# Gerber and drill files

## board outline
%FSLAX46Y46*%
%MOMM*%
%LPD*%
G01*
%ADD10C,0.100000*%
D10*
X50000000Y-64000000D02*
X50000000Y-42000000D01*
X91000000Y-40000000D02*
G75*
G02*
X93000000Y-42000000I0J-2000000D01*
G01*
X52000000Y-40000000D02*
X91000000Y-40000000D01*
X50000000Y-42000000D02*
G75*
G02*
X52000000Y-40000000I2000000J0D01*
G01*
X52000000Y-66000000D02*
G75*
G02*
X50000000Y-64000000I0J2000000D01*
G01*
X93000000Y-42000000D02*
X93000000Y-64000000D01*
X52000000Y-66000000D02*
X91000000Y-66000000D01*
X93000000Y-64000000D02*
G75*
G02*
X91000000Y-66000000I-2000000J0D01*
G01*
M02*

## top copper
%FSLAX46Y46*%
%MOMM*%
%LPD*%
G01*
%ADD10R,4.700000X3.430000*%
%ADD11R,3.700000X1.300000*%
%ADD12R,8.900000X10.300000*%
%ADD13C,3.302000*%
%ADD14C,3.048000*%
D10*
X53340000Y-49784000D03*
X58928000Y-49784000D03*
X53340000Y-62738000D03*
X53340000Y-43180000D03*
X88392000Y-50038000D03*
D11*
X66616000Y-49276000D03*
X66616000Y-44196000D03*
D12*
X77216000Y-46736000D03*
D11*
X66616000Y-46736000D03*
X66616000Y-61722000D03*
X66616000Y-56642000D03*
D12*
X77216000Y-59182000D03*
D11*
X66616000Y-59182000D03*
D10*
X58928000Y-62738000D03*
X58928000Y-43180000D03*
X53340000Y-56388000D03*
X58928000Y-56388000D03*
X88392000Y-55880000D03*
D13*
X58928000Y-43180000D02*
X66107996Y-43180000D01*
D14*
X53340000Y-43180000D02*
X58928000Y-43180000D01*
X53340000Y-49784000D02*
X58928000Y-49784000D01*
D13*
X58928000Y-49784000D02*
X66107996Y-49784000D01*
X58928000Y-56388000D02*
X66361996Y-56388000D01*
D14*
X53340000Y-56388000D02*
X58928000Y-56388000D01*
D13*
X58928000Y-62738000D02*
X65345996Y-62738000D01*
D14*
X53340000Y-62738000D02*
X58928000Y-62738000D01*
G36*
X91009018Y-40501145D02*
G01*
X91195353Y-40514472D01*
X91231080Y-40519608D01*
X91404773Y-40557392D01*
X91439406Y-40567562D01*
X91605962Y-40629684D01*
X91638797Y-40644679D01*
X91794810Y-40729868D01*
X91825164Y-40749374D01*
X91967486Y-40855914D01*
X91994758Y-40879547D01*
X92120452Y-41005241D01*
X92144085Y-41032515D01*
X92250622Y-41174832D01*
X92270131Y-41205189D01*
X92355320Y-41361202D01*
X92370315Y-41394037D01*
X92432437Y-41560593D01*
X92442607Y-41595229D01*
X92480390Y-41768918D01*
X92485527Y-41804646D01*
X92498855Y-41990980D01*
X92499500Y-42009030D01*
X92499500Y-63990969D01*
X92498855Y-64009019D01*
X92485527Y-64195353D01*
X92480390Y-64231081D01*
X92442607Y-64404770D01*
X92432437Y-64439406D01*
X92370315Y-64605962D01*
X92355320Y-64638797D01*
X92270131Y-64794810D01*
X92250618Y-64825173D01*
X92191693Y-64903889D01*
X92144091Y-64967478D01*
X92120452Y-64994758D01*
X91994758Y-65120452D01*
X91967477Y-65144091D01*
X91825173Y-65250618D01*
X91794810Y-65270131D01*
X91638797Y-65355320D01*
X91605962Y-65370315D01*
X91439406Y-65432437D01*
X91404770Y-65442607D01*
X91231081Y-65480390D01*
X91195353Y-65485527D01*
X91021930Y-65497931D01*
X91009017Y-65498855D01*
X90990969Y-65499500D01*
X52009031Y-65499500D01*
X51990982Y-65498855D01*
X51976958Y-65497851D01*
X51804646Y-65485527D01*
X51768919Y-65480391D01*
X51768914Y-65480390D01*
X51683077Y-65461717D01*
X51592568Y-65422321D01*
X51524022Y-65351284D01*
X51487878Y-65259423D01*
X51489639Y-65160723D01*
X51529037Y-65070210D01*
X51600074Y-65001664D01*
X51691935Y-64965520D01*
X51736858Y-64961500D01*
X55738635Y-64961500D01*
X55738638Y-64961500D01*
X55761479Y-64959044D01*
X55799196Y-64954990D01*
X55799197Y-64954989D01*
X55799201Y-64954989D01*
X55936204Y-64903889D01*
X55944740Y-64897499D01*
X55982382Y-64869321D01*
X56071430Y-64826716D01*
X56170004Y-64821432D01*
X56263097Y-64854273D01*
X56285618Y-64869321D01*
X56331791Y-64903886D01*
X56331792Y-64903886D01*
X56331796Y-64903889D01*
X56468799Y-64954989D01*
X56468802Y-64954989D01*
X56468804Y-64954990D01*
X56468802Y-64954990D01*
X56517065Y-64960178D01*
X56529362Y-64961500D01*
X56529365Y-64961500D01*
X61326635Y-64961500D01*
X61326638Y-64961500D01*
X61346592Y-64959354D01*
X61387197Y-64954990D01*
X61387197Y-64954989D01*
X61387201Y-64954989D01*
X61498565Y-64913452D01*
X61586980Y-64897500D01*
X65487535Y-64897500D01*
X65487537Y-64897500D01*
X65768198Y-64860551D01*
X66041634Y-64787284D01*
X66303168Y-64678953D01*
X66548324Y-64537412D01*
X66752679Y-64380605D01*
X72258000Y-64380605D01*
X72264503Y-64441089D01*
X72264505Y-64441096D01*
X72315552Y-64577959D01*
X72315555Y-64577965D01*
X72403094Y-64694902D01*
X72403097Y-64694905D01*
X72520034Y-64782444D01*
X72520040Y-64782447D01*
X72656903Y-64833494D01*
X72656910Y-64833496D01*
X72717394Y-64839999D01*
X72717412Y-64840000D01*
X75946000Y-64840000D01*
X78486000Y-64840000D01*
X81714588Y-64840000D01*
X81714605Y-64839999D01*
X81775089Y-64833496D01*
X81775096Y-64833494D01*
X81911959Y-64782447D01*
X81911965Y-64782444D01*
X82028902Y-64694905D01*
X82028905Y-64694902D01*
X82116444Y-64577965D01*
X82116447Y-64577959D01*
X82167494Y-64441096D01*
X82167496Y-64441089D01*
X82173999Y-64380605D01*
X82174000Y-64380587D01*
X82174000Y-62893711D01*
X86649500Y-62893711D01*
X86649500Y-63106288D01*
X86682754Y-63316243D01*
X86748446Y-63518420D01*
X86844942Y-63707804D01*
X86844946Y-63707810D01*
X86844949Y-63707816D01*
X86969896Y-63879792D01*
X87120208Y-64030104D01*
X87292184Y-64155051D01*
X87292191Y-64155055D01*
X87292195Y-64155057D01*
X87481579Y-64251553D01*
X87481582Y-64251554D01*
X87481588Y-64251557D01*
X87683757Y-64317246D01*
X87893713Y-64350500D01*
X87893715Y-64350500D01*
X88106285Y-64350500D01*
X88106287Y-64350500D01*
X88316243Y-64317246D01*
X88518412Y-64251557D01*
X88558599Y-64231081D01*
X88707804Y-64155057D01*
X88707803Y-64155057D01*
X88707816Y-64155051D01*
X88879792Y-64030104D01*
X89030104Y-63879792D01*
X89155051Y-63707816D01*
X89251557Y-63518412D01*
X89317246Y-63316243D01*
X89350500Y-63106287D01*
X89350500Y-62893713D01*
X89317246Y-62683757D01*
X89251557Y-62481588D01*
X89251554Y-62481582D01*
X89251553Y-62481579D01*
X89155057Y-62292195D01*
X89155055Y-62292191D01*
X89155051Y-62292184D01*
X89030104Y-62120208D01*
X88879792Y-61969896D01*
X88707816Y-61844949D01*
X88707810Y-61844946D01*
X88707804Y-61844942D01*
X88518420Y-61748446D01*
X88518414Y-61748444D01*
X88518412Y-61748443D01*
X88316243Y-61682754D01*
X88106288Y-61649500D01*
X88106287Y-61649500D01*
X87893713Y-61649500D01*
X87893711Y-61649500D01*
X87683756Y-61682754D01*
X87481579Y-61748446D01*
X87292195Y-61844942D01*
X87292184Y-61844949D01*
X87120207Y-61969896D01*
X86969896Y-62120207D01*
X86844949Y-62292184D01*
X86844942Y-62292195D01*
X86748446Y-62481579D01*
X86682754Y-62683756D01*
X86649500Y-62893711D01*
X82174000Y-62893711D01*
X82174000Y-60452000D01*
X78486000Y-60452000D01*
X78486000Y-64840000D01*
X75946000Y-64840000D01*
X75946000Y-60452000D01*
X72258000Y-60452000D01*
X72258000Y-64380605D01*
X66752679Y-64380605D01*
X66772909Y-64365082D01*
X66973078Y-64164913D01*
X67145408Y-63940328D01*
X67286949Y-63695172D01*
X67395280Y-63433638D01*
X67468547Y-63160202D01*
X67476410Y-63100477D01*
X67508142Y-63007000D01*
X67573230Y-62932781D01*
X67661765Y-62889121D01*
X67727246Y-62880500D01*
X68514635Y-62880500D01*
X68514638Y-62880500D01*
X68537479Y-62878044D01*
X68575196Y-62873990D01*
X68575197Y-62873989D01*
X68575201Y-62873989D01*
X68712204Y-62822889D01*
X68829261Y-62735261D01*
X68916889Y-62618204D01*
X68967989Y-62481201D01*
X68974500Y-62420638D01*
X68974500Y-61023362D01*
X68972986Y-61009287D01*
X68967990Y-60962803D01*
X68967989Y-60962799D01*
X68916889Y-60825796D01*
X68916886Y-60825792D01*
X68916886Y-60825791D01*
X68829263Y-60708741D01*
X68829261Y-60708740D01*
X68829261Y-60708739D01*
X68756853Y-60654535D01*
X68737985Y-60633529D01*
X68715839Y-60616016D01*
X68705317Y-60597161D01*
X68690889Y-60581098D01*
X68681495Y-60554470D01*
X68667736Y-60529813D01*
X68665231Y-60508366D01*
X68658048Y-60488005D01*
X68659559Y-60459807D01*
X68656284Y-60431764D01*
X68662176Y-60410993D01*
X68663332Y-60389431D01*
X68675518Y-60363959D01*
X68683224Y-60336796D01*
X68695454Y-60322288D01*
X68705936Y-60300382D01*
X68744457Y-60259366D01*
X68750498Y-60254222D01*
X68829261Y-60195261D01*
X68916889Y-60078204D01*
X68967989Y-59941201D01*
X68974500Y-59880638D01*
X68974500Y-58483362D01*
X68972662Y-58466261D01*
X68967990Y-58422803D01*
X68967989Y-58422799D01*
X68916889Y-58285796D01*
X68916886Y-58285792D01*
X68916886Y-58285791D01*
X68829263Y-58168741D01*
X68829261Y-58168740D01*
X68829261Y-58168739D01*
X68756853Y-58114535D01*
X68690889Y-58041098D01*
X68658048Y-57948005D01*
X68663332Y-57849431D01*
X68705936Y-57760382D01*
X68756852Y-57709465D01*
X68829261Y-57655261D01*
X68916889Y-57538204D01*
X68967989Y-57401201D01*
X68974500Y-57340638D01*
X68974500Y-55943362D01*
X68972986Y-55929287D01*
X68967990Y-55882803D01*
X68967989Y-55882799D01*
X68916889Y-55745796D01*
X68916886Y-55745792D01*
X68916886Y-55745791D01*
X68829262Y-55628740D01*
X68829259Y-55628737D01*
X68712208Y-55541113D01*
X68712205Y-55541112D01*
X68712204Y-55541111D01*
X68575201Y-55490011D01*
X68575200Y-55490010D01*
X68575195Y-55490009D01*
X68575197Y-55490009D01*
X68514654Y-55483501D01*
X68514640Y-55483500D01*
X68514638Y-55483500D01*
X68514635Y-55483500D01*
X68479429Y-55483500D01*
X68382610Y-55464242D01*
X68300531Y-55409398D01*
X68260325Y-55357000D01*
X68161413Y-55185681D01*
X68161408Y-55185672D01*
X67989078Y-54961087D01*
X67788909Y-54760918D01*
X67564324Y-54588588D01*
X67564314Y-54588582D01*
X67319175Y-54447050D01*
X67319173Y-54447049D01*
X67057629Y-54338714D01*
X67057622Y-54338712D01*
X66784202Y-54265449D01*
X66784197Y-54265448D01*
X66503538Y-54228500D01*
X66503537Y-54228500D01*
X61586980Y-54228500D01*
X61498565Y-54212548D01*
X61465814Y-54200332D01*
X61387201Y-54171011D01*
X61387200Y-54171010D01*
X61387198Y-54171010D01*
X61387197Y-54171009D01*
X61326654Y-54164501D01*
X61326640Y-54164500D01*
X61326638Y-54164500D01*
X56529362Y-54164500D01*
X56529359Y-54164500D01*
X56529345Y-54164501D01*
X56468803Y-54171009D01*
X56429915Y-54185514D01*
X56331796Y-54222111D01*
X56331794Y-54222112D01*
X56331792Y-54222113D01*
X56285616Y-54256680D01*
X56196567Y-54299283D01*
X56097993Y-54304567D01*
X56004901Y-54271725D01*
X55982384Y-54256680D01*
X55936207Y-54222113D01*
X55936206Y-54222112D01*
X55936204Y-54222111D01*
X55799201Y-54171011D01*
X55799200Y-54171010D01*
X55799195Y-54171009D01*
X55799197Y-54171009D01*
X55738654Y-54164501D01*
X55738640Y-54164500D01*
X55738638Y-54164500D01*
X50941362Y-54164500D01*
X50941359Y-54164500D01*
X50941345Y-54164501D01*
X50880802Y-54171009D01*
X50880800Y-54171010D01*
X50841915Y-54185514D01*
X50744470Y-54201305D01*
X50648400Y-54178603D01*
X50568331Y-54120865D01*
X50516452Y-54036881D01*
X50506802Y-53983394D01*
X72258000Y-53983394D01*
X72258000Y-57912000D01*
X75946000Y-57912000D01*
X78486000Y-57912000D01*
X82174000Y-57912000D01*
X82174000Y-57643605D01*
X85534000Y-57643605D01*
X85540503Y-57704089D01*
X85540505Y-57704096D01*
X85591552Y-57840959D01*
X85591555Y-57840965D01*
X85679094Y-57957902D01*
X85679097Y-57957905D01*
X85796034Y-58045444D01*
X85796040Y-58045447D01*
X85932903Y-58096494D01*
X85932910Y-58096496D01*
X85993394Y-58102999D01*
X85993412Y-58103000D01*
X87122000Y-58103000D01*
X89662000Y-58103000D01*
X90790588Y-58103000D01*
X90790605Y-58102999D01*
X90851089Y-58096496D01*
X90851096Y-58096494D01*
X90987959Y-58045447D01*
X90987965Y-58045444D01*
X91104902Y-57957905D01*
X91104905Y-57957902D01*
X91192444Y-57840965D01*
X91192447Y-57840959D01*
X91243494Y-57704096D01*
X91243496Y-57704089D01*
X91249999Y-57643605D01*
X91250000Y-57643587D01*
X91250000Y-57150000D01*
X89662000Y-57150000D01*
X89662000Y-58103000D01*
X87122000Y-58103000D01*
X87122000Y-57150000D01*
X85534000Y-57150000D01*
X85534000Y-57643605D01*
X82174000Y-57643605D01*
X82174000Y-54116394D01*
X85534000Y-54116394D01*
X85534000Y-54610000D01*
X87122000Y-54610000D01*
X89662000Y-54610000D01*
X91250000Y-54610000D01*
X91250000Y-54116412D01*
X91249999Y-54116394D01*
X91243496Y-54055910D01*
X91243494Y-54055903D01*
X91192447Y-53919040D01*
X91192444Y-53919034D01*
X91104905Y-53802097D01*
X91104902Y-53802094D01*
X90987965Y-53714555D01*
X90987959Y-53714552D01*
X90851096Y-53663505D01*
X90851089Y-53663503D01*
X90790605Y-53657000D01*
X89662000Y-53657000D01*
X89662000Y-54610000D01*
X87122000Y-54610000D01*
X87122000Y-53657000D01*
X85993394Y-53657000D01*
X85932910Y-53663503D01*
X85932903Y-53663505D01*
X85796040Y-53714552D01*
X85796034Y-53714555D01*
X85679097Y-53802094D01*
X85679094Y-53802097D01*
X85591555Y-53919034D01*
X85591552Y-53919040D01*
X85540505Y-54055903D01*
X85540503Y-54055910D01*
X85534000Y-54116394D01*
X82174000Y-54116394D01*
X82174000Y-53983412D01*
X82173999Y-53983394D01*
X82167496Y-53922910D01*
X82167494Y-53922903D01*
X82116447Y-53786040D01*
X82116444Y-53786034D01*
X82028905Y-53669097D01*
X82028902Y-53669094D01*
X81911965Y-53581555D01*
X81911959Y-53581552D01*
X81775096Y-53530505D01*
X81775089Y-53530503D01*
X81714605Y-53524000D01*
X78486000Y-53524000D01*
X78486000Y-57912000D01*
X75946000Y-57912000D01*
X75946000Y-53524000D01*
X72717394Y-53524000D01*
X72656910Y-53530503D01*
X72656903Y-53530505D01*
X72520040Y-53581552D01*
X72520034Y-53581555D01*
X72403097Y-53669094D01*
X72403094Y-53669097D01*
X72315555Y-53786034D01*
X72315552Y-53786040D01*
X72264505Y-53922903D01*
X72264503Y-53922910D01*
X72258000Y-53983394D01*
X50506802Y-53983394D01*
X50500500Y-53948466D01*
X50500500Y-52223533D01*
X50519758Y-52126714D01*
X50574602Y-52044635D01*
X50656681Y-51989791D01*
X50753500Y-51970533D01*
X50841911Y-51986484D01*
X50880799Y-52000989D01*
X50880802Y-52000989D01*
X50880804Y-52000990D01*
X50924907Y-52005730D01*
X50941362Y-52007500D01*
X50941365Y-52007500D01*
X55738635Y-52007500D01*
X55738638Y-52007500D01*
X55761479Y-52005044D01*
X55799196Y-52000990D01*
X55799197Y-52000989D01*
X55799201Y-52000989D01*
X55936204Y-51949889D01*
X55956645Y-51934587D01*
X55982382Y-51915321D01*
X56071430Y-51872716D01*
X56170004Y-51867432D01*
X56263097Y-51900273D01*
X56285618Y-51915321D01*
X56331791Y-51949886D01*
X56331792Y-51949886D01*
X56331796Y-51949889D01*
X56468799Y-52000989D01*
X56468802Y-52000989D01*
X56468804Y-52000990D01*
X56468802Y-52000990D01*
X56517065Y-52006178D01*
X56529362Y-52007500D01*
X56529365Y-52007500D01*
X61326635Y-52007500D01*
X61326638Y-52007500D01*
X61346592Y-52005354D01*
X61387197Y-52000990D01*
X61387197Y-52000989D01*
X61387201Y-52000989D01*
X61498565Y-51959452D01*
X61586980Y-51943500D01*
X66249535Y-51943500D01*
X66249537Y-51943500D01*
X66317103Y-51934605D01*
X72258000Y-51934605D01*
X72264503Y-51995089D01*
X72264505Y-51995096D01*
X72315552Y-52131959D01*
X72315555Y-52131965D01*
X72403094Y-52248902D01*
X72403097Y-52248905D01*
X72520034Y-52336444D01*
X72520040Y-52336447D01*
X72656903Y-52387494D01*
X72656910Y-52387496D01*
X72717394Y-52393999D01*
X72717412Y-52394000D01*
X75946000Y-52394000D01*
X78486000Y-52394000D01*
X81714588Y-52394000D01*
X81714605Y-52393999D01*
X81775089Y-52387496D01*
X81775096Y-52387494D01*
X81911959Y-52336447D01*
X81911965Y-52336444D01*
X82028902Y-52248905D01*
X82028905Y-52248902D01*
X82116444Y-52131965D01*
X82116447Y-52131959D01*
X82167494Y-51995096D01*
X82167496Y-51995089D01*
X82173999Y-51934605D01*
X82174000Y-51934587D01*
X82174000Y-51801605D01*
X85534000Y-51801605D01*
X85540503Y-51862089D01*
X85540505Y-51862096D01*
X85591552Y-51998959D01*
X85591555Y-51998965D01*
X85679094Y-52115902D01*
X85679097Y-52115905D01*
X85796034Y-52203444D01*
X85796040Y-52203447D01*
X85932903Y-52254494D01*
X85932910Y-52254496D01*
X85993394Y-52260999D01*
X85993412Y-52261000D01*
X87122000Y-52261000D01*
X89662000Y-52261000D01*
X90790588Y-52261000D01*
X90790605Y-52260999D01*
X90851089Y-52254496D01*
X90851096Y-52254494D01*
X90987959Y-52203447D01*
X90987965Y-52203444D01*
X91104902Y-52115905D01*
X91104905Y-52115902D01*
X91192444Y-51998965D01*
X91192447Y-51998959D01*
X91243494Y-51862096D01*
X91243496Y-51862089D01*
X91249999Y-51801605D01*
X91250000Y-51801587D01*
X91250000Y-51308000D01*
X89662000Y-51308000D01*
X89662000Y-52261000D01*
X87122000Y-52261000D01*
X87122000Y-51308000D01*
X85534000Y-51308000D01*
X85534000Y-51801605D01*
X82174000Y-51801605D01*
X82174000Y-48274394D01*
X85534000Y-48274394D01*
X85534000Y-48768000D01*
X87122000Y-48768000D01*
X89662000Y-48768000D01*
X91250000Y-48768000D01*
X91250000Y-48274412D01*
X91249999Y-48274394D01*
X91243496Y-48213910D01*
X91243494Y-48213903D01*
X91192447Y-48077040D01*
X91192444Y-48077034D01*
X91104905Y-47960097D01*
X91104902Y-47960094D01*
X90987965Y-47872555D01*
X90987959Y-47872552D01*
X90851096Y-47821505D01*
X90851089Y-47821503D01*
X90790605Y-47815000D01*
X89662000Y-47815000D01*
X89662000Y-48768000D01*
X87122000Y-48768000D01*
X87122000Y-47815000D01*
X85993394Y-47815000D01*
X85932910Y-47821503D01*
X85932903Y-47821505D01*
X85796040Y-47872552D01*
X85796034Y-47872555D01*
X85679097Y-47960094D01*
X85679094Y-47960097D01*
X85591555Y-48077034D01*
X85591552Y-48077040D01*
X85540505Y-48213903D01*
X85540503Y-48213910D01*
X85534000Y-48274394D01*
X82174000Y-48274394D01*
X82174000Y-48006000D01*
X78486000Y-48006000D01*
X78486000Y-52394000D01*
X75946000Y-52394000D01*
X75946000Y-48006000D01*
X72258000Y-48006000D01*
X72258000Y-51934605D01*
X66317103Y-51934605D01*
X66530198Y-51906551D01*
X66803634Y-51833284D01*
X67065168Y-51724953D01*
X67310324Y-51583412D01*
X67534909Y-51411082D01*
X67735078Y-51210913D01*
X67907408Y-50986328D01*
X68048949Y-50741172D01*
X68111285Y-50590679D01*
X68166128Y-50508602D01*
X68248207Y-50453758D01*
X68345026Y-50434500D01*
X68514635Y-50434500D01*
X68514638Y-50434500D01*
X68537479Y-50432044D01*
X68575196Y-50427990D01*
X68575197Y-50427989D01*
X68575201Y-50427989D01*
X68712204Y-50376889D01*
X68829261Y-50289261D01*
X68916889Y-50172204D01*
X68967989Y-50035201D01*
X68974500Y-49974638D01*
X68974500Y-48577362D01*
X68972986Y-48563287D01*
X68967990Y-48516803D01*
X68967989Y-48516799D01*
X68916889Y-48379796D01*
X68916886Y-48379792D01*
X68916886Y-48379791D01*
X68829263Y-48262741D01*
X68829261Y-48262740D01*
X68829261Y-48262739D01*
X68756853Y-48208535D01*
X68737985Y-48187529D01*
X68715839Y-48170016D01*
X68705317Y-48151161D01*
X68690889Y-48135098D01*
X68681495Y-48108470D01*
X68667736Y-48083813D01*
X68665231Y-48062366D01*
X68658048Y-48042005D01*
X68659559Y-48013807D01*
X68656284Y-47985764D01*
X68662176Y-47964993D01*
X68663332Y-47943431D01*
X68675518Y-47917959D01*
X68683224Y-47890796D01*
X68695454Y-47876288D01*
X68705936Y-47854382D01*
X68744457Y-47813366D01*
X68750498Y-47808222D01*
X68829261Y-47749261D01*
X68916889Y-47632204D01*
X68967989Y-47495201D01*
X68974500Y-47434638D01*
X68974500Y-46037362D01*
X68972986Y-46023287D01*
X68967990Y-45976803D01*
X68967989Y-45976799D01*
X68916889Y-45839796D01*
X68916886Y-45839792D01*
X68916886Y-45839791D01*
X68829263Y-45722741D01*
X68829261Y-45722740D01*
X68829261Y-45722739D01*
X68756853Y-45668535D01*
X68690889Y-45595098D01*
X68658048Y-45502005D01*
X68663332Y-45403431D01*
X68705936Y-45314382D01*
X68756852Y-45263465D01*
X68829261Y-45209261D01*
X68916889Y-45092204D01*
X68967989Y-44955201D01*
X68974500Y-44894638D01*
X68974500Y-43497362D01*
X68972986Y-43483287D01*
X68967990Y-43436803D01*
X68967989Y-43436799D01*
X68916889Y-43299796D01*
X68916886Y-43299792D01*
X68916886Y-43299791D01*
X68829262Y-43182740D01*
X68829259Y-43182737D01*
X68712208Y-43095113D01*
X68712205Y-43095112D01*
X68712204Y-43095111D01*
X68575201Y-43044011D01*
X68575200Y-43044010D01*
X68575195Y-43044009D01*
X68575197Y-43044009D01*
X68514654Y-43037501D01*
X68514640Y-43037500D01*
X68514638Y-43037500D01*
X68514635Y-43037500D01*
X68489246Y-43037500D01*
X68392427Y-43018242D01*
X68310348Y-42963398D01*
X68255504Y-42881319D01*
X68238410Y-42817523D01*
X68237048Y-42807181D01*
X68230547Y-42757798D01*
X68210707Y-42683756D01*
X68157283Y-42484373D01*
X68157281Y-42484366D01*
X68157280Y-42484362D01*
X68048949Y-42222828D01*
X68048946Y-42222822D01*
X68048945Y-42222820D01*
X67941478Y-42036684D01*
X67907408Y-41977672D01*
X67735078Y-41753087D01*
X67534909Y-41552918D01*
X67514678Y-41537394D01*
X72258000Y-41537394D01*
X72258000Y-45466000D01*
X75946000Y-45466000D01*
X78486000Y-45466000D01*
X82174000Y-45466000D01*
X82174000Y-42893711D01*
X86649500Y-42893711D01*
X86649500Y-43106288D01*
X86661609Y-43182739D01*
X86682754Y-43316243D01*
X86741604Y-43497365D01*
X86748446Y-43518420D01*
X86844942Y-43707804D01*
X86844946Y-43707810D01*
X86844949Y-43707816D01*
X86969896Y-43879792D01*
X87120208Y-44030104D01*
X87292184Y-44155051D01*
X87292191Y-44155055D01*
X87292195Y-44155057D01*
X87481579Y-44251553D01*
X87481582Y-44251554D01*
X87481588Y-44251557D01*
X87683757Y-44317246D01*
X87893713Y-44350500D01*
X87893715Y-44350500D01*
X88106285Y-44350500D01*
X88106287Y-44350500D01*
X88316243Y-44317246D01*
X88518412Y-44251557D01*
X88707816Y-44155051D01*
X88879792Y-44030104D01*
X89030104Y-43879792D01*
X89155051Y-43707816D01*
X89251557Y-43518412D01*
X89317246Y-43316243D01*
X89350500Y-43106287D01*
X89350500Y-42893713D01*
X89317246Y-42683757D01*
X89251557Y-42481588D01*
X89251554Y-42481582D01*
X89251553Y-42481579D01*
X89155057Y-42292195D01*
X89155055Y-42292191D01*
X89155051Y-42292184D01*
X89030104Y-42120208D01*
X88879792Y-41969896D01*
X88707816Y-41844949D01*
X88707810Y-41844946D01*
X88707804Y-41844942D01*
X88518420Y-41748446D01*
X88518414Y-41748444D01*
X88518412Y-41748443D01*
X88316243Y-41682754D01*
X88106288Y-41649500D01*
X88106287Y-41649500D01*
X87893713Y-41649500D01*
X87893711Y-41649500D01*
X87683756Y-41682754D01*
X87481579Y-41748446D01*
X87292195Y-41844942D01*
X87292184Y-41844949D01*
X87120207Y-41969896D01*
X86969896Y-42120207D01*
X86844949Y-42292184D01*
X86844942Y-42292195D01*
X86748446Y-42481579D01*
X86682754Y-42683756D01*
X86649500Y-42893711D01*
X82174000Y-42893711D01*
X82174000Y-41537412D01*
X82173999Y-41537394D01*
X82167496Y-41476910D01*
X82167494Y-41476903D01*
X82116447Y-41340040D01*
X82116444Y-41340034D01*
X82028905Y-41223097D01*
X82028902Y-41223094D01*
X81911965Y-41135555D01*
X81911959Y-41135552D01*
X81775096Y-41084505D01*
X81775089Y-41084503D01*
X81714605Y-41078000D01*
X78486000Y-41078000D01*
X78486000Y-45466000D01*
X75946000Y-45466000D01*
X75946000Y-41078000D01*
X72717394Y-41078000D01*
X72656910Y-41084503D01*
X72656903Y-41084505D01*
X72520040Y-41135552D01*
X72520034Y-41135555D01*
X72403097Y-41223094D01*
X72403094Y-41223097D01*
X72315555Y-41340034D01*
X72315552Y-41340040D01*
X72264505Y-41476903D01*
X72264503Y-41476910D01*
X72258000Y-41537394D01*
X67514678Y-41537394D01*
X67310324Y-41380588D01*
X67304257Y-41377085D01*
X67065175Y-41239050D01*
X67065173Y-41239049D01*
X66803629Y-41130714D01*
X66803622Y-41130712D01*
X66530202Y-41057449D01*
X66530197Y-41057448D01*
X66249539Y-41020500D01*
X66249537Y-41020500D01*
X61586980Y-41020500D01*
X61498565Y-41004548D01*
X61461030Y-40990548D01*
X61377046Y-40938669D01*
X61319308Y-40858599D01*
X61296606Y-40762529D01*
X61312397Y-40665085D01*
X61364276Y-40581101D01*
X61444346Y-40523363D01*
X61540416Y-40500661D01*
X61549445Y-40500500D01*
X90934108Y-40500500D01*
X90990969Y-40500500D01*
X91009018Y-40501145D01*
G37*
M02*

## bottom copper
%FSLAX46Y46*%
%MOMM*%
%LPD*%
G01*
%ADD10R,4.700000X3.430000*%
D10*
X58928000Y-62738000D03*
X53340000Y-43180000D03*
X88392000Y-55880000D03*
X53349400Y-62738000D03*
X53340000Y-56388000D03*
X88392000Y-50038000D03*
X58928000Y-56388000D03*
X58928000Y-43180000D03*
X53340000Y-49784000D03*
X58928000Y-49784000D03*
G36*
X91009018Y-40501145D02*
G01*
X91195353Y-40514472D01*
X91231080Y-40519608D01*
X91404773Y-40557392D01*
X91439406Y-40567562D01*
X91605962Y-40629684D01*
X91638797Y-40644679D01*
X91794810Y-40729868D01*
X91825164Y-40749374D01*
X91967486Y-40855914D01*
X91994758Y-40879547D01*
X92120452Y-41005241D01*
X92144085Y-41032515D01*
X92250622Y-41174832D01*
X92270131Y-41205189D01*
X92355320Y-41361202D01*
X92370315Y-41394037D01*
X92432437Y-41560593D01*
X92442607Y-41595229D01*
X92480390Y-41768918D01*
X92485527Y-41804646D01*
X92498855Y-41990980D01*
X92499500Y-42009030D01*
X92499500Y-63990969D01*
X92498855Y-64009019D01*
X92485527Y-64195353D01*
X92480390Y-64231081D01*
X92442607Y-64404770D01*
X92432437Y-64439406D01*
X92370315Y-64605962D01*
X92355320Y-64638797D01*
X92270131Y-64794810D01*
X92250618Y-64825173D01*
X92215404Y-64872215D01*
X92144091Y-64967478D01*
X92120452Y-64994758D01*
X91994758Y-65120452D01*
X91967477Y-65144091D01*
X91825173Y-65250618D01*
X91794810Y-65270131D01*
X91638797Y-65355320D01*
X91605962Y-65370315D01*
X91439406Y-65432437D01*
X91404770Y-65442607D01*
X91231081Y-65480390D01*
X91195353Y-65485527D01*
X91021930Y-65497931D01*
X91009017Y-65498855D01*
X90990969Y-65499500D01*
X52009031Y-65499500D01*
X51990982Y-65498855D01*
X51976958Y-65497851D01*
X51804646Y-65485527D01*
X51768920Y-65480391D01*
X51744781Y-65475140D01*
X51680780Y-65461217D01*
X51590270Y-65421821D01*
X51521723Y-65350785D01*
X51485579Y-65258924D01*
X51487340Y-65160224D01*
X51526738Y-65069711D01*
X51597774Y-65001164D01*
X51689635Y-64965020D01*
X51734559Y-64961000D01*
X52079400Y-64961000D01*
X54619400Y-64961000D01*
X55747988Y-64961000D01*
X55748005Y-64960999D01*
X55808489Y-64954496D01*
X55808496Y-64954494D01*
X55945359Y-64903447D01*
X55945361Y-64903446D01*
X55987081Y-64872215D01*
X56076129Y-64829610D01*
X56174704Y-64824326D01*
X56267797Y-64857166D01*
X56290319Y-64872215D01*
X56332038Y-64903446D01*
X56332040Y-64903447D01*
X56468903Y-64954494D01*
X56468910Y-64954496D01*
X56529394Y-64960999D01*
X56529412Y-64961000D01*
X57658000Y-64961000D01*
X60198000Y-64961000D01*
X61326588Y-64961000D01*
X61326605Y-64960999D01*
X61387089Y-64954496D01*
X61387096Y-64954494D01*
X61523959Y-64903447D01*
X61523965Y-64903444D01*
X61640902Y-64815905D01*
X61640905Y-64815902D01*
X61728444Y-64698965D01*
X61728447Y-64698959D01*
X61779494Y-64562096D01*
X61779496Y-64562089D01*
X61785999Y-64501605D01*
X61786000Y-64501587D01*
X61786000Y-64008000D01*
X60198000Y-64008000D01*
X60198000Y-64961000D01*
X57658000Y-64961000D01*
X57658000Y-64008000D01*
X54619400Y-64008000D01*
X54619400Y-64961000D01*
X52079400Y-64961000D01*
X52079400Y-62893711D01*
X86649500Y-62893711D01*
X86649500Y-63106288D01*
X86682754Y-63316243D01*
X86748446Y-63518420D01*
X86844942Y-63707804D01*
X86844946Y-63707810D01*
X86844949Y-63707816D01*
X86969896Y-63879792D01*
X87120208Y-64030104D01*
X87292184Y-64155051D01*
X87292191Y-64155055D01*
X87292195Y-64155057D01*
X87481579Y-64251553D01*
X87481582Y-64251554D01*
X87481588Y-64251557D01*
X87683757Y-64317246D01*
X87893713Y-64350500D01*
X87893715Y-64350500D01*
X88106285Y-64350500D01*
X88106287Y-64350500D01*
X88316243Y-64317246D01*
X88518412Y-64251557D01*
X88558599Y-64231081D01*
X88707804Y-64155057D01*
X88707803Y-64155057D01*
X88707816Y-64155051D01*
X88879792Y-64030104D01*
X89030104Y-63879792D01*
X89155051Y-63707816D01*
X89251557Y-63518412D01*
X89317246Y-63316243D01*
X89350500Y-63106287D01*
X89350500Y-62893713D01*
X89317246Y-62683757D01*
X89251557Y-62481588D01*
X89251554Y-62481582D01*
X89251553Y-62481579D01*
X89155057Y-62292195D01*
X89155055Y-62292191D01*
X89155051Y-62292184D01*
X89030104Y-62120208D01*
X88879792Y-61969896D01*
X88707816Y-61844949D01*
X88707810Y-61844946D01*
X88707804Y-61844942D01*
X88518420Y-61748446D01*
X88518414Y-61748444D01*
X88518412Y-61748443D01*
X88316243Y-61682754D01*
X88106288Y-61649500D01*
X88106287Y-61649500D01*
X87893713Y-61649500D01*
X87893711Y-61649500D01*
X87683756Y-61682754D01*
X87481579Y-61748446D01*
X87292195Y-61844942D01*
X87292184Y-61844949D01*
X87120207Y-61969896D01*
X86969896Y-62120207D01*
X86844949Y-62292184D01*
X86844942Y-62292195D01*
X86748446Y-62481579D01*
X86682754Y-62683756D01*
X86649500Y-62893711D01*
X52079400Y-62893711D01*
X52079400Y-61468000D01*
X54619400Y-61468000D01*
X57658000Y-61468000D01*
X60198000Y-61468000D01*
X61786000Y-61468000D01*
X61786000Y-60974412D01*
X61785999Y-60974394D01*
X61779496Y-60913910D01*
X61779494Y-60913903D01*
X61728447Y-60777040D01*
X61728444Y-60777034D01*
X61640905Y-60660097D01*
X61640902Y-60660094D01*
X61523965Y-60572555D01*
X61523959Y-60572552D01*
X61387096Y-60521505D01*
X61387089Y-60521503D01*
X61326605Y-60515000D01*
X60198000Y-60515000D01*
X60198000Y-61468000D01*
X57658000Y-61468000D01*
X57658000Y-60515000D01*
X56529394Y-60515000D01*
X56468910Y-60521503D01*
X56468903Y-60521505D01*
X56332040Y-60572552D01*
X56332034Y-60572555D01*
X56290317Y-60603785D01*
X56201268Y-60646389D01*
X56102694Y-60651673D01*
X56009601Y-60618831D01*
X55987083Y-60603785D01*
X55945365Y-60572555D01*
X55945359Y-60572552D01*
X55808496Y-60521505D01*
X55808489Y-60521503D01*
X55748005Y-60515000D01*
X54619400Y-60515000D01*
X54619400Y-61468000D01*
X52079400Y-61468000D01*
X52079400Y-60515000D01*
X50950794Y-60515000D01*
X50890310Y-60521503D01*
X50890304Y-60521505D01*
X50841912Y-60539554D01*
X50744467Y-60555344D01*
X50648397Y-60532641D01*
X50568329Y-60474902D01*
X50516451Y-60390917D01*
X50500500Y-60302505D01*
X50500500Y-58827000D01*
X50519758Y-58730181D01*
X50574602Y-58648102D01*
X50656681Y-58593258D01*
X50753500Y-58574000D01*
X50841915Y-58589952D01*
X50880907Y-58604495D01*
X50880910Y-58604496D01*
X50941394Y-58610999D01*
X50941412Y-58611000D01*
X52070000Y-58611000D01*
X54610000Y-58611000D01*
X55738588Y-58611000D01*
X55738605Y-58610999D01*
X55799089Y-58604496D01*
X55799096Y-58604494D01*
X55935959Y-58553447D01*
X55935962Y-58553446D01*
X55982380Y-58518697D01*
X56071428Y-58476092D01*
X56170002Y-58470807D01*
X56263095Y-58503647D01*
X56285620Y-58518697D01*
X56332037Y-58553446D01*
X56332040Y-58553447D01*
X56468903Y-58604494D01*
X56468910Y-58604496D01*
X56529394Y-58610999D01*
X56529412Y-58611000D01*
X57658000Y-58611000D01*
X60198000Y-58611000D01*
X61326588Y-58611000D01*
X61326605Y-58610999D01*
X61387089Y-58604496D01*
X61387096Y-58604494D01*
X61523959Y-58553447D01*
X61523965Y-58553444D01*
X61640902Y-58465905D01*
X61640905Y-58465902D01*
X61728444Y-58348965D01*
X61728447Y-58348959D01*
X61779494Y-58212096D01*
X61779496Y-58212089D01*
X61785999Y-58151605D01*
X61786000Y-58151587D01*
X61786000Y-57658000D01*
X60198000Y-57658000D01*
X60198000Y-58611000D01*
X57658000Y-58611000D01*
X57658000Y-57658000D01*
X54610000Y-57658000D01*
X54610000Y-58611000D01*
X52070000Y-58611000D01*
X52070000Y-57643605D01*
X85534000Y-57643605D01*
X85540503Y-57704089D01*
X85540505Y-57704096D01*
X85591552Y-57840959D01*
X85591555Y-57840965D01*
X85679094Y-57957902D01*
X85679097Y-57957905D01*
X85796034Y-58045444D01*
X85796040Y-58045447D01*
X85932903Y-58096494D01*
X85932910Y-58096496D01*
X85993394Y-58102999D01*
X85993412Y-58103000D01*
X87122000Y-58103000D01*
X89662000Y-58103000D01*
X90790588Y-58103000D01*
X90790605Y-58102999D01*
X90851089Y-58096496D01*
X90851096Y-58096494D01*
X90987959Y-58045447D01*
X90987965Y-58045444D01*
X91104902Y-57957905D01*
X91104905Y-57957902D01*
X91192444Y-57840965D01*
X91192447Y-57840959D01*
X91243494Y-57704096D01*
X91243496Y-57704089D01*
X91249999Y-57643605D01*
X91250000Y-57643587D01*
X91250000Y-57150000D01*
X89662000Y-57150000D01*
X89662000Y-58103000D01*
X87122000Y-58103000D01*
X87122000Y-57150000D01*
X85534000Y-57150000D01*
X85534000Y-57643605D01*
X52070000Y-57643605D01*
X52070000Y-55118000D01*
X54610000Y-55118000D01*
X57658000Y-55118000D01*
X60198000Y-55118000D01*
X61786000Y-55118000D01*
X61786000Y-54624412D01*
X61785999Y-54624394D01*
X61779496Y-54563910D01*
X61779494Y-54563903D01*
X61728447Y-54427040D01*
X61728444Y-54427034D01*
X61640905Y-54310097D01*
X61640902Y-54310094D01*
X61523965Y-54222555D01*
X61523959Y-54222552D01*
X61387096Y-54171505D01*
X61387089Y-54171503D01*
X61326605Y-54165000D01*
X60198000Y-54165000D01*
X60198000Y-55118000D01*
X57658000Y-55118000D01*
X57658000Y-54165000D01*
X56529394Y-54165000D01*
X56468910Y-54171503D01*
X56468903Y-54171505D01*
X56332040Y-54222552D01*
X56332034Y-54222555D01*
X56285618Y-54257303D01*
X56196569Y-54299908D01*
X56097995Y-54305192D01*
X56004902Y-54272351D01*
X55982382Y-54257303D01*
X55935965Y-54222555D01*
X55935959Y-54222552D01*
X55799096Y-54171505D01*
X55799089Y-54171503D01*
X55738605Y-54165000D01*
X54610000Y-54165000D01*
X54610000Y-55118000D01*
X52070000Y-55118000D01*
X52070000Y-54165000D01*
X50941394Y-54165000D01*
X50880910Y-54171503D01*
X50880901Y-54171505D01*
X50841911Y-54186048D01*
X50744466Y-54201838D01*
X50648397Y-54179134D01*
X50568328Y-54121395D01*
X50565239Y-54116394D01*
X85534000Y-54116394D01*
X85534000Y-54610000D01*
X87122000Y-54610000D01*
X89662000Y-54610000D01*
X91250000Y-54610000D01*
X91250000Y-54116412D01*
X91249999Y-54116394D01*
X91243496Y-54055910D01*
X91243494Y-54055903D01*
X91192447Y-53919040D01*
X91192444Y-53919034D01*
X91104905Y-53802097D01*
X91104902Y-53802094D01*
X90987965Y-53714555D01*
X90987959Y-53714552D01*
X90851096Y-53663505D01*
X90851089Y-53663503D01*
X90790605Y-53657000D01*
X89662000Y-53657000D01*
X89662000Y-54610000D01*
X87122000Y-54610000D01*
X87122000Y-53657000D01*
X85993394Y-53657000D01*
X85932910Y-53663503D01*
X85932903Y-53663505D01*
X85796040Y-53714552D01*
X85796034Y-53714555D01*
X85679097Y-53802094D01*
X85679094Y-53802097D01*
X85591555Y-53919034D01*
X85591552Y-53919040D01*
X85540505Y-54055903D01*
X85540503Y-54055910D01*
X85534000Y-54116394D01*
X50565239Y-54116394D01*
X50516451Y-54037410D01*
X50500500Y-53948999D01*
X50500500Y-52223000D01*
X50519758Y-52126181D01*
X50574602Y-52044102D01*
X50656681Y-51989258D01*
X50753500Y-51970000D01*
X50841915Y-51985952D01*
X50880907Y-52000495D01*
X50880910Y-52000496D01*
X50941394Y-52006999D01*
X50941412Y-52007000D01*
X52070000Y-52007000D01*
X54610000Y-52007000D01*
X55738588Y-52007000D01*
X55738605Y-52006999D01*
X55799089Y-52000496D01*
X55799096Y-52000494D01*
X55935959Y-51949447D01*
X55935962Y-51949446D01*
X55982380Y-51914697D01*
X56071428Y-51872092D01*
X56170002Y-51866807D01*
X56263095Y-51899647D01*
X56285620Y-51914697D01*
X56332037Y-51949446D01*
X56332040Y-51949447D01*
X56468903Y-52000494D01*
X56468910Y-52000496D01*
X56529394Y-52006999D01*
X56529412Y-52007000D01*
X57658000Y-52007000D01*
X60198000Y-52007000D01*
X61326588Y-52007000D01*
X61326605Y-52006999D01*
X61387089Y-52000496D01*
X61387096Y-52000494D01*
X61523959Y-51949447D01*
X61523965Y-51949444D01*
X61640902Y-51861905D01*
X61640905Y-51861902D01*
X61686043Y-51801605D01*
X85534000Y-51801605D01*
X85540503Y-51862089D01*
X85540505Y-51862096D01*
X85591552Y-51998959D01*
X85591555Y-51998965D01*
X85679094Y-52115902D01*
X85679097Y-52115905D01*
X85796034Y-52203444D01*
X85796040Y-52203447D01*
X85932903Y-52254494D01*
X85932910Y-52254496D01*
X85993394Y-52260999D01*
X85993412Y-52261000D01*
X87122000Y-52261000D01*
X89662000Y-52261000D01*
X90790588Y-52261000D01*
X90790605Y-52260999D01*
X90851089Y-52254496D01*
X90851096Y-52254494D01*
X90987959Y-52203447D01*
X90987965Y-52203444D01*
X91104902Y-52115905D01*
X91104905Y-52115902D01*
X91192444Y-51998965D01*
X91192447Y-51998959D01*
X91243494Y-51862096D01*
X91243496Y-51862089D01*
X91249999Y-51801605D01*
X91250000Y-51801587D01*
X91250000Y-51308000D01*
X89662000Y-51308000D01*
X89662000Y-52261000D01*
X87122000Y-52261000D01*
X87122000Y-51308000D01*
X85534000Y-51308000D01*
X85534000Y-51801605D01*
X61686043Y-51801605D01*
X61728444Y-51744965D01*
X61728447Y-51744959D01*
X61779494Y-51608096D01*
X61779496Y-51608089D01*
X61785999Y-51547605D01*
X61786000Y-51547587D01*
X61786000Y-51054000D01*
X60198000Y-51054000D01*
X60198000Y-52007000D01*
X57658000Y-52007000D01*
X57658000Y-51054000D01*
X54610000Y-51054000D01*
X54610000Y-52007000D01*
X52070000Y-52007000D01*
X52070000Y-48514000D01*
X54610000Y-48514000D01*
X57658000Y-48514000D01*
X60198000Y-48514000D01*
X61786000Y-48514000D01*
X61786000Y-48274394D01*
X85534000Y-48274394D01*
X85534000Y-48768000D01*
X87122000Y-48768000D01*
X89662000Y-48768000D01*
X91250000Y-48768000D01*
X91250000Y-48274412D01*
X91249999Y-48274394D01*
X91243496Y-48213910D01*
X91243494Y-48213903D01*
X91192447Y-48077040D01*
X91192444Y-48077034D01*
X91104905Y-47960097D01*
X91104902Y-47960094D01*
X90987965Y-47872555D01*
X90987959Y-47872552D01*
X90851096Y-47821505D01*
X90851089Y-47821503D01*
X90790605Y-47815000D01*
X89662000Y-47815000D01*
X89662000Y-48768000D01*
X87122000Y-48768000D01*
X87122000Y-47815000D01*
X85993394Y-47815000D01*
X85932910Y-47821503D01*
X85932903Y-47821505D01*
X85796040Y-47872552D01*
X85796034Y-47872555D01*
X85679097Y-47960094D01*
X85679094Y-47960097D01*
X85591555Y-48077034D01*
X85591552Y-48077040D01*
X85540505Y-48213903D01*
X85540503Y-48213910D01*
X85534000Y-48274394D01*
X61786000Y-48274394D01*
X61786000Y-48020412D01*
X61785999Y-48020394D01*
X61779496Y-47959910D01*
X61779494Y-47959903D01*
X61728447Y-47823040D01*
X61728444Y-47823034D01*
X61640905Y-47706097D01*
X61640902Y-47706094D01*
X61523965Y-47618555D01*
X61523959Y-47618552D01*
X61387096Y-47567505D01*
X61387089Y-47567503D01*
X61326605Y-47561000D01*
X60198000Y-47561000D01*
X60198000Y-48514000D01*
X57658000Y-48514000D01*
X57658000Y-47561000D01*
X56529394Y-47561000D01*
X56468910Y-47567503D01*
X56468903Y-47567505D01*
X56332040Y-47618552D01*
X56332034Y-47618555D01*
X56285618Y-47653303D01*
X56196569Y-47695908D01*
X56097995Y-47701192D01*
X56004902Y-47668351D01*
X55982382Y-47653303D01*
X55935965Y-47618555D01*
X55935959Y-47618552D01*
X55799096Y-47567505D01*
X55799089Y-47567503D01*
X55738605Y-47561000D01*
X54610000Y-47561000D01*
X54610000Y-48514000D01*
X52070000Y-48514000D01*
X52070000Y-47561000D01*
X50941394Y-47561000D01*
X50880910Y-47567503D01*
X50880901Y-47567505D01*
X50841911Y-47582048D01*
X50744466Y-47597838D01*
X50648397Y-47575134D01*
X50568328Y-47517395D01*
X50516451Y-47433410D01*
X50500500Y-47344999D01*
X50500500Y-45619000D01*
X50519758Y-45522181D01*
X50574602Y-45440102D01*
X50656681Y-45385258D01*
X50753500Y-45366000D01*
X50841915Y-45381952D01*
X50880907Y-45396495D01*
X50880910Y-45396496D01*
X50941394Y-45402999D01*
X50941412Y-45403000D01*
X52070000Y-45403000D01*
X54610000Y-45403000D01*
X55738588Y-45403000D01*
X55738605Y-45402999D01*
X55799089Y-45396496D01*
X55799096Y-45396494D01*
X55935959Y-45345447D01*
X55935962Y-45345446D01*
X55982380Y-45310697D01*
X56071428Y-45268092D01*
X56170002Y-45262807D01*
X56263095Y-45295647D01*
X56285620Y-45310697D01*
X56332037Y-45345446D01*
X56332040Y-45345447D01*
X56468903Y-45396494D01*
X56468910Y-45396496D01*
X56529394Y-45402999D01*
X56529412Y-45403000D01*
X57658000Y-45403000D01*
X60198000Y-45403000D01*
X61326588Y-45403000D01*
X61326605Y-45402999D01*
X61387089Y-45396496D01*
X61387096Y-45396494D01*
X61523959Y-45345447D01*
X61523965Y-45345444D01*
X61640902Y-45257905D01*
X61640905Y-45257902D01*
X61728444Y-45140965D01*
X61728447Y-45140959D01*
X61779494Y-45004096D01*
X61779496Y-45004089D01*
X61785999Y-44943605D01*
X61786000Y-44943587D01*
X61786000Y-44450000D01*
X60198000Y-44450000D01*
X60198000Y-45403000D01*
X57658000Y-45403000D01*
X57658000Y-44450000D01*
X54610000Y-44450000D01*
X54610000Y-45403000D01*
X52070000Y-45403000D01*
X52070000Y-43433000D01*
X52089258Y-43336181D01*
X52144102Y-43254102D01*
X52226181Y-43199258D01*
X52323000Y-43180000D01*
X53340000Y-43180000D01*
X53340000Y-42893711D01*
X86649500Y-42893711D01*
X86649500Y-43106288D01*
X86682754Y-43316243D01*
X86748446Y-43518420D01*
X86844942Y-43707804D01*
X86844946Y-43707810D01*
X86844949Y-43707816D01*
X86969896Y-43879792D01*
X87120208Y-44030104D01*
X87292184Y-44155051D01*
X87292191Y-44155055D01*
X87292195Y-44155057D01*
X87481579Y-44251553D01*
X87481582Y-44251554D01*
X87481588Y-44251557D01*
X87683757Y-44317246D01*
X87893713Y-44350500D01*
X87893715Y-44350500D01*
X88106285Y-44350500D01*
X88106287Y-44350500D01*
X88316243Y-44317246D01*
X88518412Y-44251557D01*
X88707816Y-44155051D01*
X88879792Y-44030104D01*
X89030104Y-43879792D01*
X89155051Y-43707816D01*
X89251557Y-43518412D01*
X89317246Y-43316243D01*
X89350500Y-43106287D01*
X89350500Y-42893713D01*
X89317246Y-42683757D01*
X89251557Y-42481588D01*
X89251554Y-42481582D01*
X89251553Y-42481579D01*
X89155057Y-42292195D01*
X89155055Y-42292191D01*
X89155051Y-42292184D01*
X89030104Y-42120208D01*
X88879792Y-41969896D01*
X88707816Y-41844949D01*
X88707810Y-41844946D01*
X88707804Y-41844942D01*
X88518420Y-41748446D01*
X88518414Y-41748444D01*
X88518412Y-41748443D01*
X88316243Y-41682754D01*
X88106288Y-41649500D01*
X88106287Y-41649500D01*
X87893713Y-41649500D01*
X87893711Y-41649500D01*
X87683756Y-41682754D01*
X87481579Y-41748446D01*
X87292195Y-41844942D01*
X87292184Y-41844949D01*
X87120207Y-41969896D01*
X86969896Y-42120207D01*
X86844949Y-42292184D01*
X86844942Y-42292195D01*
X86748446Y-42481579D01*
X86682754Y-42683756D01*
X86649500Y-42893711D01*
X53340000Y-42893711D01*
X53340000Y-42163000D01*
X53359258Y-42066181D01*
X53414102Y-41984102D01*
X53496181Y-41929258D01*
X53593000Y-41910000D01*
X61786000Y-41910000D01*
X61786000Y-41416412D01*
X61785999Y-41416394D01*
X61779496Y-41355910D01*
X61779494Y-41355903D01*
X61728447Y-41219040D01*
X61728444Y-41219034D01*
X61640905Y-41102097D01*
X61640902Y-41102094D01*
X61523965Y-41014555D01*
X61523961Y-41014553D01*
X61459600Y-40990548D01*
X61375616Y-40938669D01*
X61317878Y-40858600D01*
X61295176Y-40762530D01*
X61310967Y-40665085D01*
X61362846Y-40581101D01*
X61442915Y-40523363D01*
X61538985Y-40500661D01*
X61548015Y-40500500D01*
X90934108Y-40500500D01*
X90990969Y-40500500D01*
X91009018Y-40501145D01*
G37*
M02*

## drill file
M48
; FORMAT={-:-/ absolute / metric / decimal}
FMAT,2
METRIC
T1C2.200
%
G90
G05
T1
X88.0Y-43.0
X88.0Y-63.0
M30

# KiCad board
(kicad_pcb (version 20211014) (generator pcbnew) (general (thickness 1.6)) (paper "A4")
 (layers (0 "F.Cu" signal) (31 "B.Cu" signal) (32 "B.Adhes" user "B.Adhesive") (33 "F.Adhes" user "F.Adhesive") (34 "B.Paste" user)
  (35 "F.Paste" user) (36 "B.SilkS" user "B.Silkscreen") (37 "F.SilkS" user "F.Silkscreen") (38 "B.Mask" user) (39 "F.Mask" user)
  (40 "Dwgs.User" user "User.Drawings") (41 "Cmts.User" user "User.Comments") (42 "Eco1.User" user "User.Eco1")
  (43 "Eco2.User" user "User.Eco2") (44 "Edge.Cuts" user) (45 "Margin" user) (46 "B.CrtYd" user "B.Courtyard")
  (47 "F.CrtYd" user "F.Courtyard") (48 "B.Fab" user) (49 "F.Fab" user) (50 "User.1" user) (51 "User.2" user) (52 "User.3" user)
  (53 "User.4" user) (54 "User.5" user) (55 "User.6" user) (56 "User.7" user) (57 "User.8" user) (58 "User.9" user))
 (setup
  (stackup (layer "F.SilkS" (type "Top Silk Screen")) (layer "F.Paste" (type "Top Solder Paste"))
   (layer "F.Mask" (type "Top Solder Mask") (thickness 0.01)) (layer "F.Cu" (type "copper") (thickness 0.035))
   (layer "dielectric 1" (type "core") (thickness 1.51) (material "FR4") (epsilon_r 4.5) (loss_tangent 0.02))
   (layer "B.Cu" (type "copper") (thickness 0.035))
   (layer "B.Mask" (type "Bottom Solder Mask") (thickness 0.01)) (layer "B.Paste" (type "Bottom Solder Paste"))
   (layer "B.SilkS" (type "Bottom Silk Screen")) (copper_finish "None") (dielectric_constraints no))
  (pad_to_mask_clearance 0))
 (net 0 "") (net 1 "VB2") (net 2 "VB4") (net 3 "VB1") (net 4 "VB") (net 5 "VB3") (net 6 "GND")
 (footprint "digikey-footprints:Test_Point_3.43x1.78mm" (layer "F.Cu") (at 53.34 49.784)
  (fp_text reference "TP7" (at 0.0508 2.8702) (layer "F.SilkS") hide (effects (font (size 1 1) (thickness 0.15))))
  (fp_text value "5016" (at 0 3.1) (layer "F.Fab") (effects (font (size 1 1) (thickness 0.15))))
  (pad "1" smd rect locked (at 0 0) (size 4.7 3.43) (layers "F.Cu" "F.Paste" "F.Mask") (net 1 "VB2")))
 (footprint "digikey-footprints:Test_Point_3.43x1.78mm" (layer "F.Cu") (at 58.928 49.784 180)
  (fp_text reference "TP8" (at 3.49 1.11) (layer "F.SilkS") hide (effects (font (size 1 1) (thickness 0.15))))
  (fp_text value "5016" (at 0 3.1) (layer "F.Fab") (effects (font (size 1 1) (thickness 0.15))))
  (pad "1" smd rect locked (at 0 0 180) (size 4.7 3.43) (layers "F.Cu" "F.Paste" "F.Mask") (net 1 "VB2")))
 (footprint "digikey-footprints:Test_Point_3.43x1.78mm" (layer "F.Cu") (at 53.34 62.738)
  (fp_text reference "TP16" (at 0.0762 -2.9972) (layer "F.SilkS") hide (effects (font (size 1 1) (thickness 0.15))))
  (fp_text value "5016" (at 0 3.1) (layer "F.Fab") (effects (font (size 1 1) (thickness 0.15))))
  (pad "1" smd rect locked (at 0 0) (size 4.7 3.43) (layers "F.Cu" "F.Paste" "F.Mask") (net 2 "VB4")))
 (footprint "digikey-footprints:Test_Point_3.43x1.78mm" (layer "F.Cu") (at 53.34 43.18)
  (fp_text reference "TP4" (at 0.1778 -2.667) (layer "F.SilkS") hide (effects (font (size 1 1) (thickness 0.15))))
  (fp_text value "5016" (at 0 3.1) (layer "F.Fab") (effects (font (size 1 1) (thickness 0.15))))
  (pad "1" smd rect locked (at 0 0) (size 4.7 3.43) (layers "F.Cu" "F.Paste" "F.Mask") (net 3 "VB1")))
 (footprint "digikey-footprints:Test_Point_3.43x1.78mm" (layer "F.Cu") (at 88.392 50.038 180)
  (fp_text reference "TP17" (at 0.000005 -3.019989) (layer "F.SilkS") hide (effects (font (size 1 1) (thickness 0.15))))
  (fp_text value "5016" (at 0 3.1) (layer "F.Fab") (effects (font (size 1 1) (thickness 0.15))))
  (pad "1" smd rect locked (at 0 0 180) (size 4.7 3.43) (layers "F.Cu" "F.Paste" "F.Mask") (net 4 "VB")))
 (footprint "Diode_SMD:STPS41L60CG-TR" (layer "F.Cu") (at 77.216 46.736 180)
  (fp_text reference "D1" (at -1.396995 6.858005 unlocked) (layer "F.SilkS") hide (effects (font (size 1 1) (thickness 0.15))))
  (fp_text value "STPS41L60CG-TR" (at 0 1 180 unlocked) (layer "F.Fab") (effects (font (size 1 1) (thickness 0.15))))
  (pad "1" smd rect (at 10.6 -2.54 180) (size 3.7 1.3) (layers "F.Cu" "F.Paste" "F.Mask") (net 1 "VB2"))
  (pad "2" smd rect (at 10.6 2.54 180) (size 3.7 1.3) (layers "F.Cu" "F.Paste" "F.Mask") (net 3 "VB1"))
  (pad "3" smd rect (at 0 0 180) (size 8.9 10.3) (layers "F.Cu" "F.Paste" "F.Mask") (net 4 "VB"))
  (pad "4" smd rect (at 10.6 0 180) (size 3.7 1.3) (layers "F.Cu" "F.Paste" "F.Mask")))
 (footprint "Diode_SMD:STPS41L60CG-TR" (layer "F.Cu") (at 77.216 59.182 180)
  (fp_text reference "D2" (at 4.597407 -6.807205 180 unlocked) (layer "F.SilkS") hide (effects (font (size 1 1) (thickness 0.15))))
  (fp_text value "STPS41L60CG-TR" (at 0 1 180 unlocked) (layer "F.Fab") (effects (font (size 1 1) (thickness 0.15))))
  (pad "1" smd rect (at 10.6 -2.54 180) (size 3.7 1.3) (layers "F.Cu" "F.Paste" "F.Mask") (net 2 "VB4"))
  (pad "2" smd rect (at 10.6 2.54 180) (size 3.7 1.3) (layers "F.Cu" "F.Paste" "F.Mask") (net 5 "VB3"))
  (pad "3" smd rect (at 0 0 180) (size 8.9 10.3) (layers "F.Cu" "F.Paste" "F.Mask") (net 4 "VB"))
  (pad "4" smd rect (at 10.6 0 180) (size 3.7 1.3) (layers "F.Cu" "F.Paste" "F.Mask")))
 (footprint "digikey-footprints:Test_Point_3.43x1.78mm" (layer "F.Cu") (at 58.928 62.738)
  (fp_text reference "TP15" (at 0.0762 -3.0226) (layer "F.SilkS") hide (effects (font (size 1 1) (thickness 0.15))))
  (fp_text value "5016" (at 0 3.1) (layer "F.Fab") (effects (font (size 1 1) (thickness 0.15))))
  (pad "1" smd rect locked (at 0 0) (size 4.7 3.43) (layers "F.Cu" "F.Paste" "F.Mask") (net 2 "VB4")))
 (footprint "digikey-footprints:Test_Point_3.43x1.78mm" (layer "F.Cu") (at 58.928 43.18 180)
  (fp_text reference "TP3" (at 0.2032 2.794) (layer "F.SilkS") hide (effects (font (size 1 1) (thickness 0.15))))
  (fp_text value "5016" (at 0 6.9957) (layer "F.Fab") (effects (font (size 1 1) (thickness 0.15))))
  (pad "1" smd rect locked (at 0 0 180) (size 4.7 3.43) (layers "F.Cu" "F.Paste" "F.Mask") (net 3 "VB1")))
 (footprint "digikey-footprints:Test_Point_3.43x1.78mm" (layer "F.Cu") (at 53.34 56.388)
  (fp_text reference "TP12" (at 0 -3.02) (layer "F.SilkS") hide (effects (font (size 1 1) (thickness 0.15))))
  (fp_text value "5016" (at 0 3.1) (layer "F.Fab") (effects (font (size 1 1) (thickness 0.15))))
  (pad "1" smd rect locked (at 0 0) (size 4.7 3.43) (layers "F.Cu" "F.Paste" "F.Mask") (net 5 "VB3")))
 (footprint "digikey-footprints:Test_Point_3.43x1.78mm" (layer "F.Cu") (at 58.928 56.388)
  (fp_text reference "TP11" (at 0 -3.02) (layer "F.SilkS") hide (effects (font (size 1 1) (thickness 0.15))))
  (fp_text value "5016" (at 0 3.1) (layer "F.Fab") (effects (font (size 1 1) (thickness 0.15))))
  (pad "1" smd rect locked (at 0 0) (size 4.7 3.43) (layers "F.Cu" "F.Paste" "F.Mask") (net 5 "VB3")))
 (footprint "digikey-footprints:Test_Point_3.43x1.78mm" (layer "F.Cu") (at 88.392 55.88 180)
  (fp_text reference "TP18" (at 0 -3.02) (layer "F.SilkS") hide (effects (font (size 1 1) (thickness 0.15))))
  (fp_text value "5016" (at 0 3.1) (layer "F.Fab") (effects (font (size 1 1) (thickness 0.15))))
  (pad "1" smd rect locked (at 0 0 180) (size 4.7 3.43) (layers "F.Cu" "F.Paste" "F.Mask") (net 4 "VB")))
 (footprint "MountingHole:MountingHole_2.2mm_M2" (layer "F.Cu") (at 88 43)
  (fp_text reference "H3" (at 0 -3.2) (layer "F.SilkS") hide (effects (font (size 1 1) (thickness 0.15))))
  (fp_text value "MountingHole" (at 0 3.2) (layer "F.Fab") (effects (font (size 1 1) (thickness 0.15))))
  (pad "" np_thru_hole circle (at 0 0) (size 2.2 2.2) (drill 2.2) (layers *.Cu *.Mask)))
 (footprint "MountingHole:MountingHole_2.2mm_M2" (layer "F.Cu") (at 88 63)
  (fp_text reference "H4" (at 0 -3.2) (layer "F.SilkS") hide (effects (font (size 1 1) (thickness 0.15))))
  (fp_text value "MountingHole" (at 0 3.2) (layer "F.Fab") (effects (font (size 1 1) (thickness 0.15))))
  (pad "" np_thru_hole circle (at 0 0) (size 2.2 2.2) (drill 2.2) (layers *.Cu *.Mask)))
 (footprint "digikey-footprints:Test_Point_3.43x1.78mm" (layer "B.Cu") (at 58.928 62.738 180)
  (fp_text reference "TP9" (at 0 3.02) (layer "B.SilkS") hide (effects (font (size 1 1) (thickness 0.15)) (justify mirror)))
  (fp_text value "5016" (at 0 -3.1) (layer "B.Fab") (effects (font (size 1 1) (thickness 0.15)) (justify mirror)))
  (pad "1" smd rect locked (at 0 0 180) (size 4.7 3.43) (layers "B.Cu" "B.Paste" "B.Mask") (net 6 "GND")))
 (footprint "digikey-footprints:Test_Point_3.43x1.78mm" (layer "B.Cu") (at 53.34 43.18 180)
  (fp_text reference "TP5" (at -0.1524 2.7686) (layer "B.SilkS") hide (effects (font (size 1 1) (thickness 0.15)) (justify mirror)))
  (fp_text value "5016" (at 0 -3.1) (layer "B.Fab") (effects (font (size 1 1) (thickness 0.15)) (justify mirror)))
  (pad "1" smd rect locked (at 0 0 180) (size 4.7 3.43) (layers "B.Cu" "B.Paste" "B.Mask") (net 6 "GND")))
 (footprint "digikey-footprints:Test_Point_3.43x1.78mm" (layer "B.Cu") (at 88.392 55.88 180)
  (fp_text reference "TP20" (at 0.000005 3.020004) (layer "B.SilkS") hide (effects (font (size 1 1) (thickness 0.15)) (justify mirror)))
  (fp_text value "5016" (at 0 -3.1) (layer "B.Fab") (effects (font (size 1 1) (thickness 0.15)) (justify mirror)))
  (pad "1" smd rect locked (at 0 0 180) (size 4.7 3.43) (layers "B.Cu" "B.Paste" "B.Mask") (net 6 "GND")))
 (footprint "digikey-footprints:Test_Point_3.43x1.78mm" (layer "B.Cu") (at 53.3494 62.738)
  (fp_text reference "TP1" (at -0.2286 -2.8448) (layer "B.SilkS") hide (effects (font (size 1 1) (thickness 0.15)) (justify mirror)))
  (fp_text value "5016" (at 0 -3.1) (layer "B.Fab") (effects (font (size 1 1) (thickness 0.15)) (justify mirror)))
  (pad "1" smd rect locked (at 0 0) (size 4.7 3.43) (layers "B.Cu" "B.Paste" "B.Mask") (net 6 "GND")))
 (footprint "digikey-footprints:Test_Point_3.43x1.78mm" (layer "B.Cu") (at 53.34 56.388)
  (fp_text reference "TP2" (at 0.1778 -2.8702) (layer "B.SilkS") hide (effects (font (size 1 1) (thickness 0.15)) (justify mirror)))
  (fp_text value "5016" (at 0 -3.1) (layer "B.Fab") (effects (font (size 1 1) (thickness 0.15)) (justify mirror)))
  (pad "1" smd rect locked (at 0 0) (size 4.7 3.43) (layers "B.Cu" "B.Paste" "B.Mask") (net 6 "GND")))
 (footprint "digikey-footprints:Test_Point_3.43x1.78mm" (layer "B.Cu") (at 88.392 50.038 180)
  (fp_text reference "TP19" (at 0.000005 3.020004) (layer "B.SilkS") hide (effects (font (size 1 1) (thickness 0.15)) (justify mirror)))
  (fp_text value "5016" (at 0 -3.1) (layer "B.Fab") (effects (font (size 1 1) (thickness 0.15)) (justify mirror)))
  (pad "1" smd rect locked (at 0 0 180) (size 4.7 3.43) (layers "B.Cu" "B.Paste" "B.Mask") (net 6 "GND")))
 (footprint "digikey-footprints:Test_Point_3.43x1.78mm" (layer "B.Cu") (at 58.928 56.388 180)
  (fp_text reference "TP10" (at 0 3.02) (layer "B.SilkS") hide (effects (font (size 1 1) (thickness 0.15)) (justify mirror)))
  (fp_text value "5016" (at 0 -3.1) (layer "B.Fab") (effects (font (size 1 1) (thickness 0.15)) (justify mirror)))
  (pad "1" smd rect locked (at 0 0 180) (size 4.7 3.43) (layers "B.Cu" "B.Paste" "B.Mask") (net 6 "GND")))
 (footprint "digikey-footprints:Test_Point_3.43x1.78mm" (layer "B.Cu") (at 58.928 43.18 180)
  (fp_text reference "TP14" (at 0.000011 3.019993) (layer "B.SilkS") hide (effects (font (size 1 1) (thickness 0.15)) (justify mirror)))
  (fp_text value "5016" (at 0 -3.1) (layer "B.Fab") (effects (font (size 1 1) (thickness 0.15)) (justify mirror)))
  (pad "1" smd rect locked (at 0 0 180) (size 4.7 3.43) (layers "B.Cu" "B.Paste" "B.Mask") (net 6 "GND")))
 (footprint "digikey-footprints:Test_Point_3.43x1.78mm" (layer "B.Cu") (at 53.34 49.784 180)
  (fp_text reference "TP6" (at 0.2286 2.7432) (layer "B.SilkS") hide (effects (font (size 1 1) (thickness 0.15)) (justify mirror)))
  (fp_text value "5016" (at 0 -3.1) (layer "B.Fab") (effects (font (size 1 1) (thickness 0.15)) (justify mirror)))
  (pad "1" smd rect locked (at 0 0 180) (size 4.7 3.43) (layers "B.Cu" "B.Paste" "B.Mask") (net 6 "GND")))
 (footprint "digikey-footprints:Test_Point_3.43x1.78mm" (layer "B.Cu") (at 58.928 49.784 180)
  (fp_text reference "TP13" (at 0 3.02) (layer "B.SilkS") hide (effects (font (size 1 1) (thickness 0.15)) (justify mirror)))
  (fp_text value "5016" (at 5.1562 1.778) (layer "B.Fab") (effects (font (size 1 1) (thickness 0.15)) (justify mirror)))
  (pad "1" smd rect locked (at 0 0 180) (size 4.7 3.43) (layers "B.Cu" "B.Paste" "B.Mask") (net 6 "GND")))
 (gr_line (start 50 64) (end 50 42) (layer "Edge.Cuts") (width 0.1))
 (gr_arc (start 91 40) (mid 92.414214 40.585786) (end 93 42) (layer "Edge.Cuts") (width 0.1))
 (gr_line (start 52 40) (end 91 40) (layer "Edge.Cuts") (width 0.1))
 (gr_arc (start 50 42) (mid 50.585786 40.585786) (end 52 40) (layer "Edge.Cuts") (width 0.1))
 (gr_arc (start 52 66) (mid 50.585786 65.414214) (end 50 64) (layer "Edge.Cuts") (width 0.1))
 (gr_line (start 93 42) (end 93 64) (layer "Edge.Cuts") (width 0.1))
 (gr_line (start 52 66) (end 91 66) (layer "Edge.Cuts") (width 0.1))
 (gr_arc (start 93 64) (mid 92.414214 65.414214) (end 91 66) (layer "Edge.Cuts") (width 0.1))
 (segment (start 58.928 43.18) (end 66.107996 43.18) (width 3.302) (layer "F.Cu") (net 3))
 (segment (start 53.34 43.18) (end 58.928 43.18) (width 3.048) (layer "F.Cu") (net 3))
 (segment (start 53.34 49.784) (end 58.928 49.784) (width 3.048) (layer "F.Cu") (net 1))
 (segment (start 58.928 49.784) (end 66.107996 49.784) (width 3.302) (layer "F.Cu") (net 1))
 (segment (start 58.928 56.388) (end 66.361996 56.388) (width 3.302) (layer "F.Cu") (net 5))
 (segment (start 53.34 56.388) (end 58.928 56.388) (width 3.048) (layer "F.Cu") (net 5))
 (segment (start 58.928 62.738) (end 65.345996 62.738) (width 3.302) (layer "F.Cu") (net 2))
 (segment (start 53.34 62.738) (end 58.928 62.738) (width 3.048) (layer "F.Cu") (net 2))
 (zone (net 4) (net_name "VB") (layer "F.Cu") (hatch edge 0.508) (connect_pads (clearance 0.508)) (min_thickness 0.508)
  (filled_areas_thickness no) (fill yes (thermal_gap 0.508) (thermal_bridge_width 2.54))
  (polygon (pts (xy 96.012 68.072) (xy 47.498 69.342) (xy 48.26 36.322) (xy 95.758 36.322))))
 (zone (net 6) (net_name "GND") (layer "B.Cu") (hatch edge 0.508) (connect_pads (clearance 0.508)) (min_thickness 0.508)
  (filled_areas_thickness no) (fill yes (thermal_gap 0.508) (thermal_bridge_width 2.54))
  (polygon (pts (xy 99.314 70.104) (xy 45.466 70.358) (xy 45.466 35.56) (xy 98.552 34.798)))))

